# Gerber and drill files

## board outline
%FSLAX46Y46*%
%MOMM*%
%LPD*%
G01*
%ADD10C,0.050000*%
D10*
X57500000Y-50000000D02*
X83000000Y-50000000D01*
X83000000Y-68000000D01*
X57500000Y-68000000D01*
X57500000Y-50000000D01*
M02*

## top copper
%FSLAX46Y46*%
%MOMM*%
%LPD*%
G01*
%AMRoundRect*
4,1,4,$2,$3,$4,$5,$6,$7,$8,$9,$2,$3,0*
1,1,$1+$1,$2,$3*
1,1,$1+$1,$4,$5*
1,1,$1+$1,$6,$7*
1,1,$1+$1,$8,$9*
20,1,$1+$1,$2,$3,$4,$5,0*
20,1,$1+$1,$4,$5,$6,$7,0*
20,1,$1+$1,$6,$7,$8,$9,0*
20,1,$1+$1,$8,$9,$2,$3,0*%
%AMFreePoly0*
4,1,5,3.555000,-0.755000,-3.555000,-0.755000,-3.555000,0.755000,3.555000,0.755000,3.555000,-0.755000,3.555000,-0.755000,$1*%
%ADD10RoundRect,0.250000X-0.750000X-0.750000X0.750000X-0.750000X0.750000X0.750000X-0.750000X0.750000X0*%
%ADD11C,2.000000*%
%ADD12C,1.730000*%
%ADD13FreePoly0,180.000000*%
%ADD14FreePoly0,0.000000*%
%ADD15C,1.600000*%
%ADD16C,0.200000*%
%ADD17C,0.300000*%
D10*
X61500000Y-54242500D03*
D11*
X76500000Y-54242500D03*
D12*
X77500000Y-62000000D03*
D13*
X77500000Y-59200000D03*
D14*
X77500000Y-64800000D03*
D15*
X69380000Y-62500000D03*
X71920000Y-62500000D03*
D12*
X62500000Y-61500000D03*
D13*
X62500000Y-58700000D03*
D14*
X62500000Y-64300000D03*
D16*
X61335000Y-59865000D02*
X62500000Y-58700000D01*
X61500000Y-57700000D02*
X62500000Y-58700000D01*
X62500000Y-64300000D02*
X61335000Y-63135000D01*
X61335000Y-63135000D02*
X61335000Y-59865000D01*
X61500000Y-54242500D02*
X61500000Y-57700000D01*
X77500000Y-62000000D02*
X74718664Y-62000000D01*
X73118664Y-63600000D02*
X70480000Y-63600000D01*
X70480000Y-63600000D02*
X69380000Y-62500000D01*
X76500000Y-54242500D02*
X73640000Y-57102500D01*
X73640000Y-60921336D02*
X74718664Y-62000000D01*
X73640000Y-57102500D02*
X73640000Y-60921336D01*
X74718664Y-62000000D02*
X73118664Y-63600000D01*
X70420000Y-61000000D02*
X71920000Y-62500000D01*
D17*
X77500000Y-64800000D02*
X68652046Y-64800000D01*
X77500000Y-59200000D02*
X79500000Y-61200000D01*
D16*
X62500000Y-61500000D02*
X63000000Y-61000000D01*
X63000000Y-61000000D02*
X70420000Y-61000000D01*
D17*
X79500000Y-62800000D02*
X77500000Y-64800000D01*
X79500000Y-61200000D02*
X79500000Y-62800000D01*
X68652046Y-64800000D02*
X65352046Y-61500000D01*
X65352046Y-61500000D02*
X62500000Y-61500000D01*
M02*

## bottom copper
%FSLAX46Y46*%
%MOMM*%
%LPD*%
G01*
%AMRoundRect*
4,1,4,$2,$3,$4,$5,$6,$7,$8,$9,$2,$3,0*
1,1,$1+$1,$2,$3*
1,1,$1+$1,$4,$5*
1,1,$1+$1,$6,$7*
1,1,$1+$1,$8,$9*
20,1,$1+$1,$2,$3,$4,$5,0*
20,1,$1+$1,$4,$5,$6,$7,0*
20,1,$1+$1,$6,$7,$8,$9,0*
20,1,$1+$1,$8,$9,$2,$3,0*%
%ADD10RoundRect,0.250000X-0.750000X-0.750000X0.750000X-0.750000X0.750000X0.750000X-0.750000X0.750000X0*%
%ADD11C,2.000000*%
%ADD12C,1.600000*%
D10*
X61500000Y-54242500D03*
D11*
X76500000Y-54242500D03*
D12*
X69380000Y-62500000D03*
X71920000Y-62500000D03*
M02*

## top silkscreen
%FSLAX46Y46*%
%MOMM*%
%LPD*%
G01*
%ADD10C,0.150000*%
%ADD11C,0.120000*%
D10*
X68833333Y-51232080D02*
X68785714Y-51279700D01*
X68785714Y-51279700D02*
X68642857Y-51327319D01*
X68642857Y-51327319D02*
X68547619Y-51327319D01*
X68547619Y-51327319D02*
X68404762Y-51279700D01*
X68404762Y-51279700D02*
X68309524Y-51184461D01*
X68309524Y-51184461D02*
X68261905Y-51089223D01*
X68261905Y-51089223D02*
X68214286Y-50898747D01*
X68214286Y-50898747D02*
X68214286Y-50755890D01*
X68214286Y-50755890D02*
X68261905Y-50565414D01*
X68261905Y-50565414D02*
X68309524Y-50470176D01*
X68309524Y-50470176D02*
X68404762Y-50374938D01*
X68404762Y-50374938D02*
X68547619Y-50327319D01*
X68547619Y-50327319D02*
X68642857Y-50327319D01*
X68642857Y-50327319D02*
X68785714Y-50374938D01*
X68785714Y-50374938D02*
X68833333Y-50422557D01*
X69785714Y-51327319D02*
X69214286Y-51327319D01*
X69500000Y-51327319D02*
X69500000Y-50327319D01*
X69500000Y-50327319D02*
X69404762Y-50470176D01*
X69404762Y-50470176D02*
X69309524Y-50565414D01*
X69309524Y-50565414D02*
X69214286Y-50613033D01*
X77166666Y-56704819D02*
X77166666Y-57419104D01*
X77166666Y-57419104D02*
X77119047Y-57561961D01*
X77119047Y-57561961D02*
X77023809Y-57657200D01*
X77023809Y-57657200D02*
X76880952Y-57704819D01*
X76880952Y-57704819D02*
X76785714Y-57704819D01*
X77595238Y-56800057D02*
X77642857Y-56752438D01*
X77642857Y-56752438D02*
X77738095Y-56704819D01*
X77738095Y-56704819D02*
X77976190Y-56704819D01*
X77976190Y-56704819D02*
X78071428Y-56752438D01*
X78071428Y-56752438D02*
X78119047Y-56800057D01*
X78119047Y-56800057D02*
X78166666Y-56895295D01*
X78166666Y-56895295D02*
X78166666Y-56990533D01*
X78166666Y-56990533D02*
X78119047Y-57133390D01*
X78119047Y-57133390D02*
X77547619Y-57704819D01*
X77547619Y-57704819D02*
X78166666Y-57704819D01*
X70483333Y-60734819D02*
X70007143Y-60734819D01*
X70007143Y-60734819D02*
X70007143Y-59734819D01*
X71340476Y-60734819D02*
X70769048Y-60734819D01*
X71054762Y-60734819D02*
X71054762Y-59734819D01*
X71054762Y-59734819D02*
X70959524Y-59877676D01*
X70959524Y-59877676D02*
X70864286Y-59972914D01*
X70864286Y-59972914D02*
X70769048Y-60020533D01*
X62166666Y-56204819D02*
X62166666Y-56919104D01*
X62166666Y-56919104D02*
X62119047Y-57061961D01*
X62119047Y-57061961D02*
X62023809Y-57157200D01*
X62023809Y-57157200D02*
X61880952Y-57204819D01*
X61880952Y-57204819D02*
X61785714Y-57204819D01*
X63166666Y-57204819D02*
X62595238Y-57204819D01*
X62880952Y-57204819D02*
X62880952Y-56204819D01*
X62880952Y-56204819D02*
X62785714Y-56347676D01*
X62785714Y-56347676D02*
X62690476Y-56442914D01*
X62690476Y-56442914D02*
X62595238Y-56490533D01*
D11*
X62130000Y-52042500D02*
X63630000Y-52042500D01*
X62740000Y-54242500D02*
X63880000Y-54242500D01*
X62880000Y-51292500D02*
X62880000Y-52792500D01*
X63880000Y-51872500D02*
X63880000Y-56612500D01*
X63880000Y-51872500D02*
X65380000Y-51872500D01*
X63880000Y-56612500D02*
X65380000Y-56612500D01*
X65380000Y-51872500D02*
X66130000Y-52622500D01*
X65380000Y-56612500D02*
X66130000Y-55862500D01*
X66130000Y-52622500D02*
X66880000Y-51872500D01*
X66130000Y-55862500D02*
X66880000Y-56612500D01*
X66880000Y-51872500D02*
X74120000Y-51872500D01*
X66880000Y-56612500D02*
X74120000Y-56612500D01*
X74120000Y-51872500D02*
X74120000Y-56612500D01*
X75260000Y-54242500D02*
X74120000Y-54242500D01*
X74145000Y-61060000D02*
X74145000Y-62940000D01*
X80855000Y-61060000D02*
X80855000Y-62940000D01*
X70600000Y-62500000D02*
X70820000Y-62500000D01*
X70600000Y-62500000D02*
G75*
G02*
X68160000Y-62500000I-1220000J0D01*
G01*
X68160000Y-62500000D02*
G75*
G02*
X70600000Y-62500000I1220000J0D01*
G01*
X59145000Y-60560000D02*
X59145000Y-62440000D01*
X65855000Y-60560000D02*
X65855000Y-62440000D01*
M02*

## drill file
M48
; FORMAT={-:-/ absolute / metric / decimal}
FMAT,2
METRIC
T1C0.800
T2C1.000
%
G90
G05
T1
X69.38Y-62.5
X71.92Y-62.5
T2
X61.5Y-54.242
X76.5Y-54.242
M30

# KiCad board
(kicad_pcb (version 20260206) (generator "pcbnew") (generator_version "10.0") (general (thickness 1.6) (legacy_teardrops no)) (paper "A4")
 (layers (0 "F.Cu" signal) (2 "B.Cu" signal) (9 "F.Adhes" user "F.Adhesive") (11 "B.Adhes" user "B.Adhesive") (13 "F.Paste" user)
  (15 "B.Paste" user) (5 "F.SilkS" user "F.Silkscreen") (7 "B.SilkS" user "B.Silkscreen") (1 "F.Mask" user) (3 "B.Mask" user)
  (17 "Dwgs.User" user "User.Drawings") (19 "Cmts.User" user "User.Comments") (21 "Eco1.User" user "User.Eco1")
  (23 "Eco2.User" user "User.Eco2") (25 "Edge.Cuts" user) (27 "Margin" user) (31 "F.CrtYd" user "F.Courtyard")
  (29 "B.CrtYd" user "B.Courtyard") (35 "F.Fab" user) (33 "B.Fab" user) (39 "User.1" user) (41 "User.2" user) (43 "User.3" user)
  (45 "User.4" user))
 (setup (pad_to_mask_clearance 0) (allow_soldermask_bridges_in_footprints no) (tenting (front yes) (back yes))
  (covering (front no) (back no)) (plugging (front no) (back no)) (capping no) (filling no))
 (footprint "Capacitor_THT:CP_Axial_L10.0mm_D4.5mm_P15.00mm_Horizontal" (layer "F.Cu") (at 61.5 54.2425)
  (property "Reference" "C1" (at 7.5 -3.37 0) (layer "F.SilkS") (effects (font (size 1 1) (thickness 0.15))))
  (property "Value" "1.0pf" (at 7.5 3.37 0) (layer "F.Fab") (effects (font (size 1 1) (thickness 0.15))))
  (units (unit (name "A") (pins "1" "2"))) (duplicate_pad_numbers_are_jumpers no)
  (fp_line (start 0.63 -2.2) (end 2.13 -2.2) (stroke (width 0.12) (type solid)) (layer "F.SilkS"))
  (fp_line (start 1.24 0) (end 2.38 0) (stroke (width 0.12) (type solid)) (layer "F.SilkS"))
  (fp_line (start 1.38 -2.95) (end 1.38 -1.45) (stroke (width 0.12) (type solid)) (layer "F.SilkS"))
  (fp_line (start 2.38 -2.37) (end 2.38 2.37) (stroke (width 0.12) (type solid)) (layer "F.SilkS"))
  (fp_line (start 2.38 -2.37) (end 3.88 -2.37) (stroke (width 0.12) (type solid)) (layer "F.SilkS"))
  (fp_line (start 2.38 2.37) (end 3.88 2.37) (stroke (width 0.12) (type solid)) (layer "F.SilkS"))
  (fp_line (start 3.88 -2.37) (end 4.63 -1.62) (stroke (width 0.12) (type solid)) (layer "F.SilkS"))
  (fp_line (start 3.88 2.37) (end 4.63 1.62) (stroke (width 0.12) (type solid)) (layer "F.SilkS"))
  (fp_line (start 4.63 -1.62) (end 5.38 -2.37) (stroke (width 0.12) (type solid)) (layer "F.SilkS"))
  (fp_line (start 4.63 1.62) (end 5.38 2.37) (stroke (width 0.12) (type solid)) (layer "F.SilkS"))
  (fp_line (start 5.38 -2.37) (end 12.62 -2.37) (stroke (width 0.12) (type solid)) (layer "F.SilkS"))
  (fp_line (start 5.38 2.37) (end 12.62 2.37) (stroke (width 0.12) (type solid)) (layer "F.SilkS"))
  (fp_line (start 12.62 -2.37) (end 12.62 2.37) (stroke (width 0.12) (type solid)) (layer "F.SilkS"))
  (fp_line (start 13.76 0) (end 12.62 0) (stroke (width 0.12) (type solid)) (layer "F.SilkS"))
  (pad "1" thru_hole roundrect (at 0 0) (size 2 2) (drill 1) (layers "*.Cu" "*.Mask") (remove_unused_layers no) (roundrect_rratio 0.125)
   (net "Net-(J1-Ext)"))
  (pad "2" thru_hole circle (at 15 0) (size 2 2) (drill 1) (layers "*.Cu" "*.Mask") (remove_unused_layers no) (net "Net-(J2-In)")))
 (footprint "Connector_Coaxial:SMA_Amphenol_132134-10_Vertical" (layer "F.Cu") (at 77.5 62)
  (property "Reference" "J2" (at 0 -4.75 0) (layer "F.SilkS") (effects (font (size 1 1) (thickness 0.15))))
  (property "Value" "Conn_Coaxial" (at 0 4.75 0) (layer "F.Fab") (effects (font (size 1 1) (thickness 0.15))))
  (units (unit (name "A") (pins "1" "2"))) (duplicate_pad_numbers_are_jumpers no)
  (fp_line (start -3.355 -0.94) (end -3.355 0.94) (stroke (width 0.12) (type solid)) (layer "F.SilkS"))
  (fp_line (start 3.355 -0.94) (end 3.355 0.94) (stroke (width 0.12) (type solid)) (layer "F.SilkS"))
  (pad "1" smd circle (at 0 0 90) (size 1.73 1.73) (layers "F.Cu" "F.Mask" "F.Paste") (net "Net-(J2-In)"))
  (pad "2" smd custom (at 0 -2.8 180) (size 7.11 1.51) (layers "F.Cu" "F.Mask" "F.Paste") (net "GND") (zone_connect 2)
   (options (clearance outline) (anchor rect)) (primitives))
  (pad "2" smd custom (at 0 2.8) (size 7.11 1.51) (layers "F.Cu" "F.Mask" "F.Paste") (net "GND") (zone_connect 2)
   (options (clearance outline) (anchor rect)) (primitives)))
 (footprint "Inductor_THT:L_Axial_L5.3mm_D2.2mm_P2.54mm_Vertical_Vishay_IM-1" (layer "F.Cu") (at 69.38 62.5)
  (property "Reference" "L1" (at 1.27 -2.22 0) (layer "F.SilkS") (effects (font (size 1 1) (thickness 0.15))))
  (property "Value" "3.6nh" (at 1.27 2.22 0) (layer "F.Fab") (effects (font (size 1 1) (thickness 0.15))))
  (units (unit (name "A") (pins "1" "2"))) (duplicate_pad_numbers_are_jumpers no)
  (fp_line (start 1.22 0) (end 1.44 0) (stroke (width 0.12) (type solid)) (layer "F.SilkS"))
  (fp_circle (center 0 0) (end 1.22 0) (stroke (width 0.12) (type solid)) (fill no) (layer "F.SilkS"))
  (pad "1" thru_hole circle (at 0 0) (size 1.6 1.6) (drill 0.8) (layers "*.Cu" "*.Mask") (remove_unused_layers no) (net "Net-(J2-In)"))
  (pad "2" thru_hole circle (at 2.54 0) (size 1.6 1.6) (drill 0.8) (layers "*.Cu" "*.Mask") (remove_unused_layers no) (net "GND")))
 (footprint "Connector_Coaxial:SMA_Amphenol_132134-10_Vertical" (layer "F.Cu") (at 62.5 61.5)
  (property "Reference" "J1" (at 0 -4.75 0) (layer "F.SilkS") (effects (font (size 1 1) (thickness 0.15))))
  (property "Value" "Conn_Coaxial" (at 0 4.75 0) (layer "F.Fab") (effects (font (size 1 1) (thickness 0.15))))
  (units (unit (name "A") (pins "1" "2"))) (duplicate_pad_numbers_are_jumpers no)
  (fp_line (start -3.355 -0.94) (end -3.355 0.94) (stroke (width 0.12) (type solid)) (layer "F.SilkS"))
  (fp_line (start 3.355 -0.94) (end 3.355 0.94) (stroke (width 0.12) (type solid)) (layer "F.SilkS"))
  (pad "1" smd circle (at 0 0 90) (size 1.73 1.73) (layers "F.Cu" "F.Mask" "F.Paste") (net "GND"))
  (pad "2" smd custom (at 0 -2.8 180) (size 7.11 1.51) (layers "F.Cu" "F.Mask" "F.Paste") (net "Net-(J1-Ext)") (zone_connect 2)
   (options (clearance outline) (anchor rect)) (primitives))
  (pad "2" smd custom (at 0 2.8) (size 7.11 1.51) (layers "F.Cu" "F.Mask" "F.Paste") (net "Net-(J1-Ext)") (zone_connect 2)
   (options (clearance outline) (anchor rect)) (primitives)))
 (gr_rect (start 57.5 50) (end 83 68) (stroke (width 0.05) (type default)) (fill no) (layer "Edge.Cuts"))
 (segment (start 61.335 59.865) (end 62.5 58.7) (width 0.2) (layer "F.Cu") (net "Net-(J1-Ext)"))
 (segment (start 61.5 57.7) (end 62.5 58.7) (width 0.2) (layer "F.Cu") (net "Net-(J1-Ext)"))
 (segment (start 62.5 64.3) (end 61.335 63.135) (width 0.2) (layer "F.Cu") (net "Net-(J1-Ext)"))
 (segment (start 61.335 63.135) (end 61.335 59.865) (width 0.2) (layer "F.Cu") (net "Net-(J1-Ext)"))
 (segment (start 61.5 54.2425) (end 61.5 57.7) (width 0.2) (layer "F.Cu") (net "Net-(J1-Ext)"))
 (segment (start 77.5 62) (end 74.718664 62) (width 0.2) (layer "F.Cu") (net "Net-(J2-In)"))
 (segment (start 73.118664 63.6) (end 70.48 63.6) (width 0.2) (layer "F.Cu") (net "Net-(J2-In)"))
 (segment (start 70.48 63.6) (end 69.38 62.5) (width 0.2) (layer "F.Cu") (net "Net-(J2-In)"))
 (segment (start 76.5 54.2425) (end 73.64 57.1025) (width 0.2) (layer "F.Cu") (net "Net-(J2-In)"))
 (segment (start 73.64 60.921336) (end 74.718664 62) (width 0.2) (layer "F.Cu") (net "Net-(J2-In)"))
 (segment (start 73.64 57.1025) (end 73.64 60.921336) (width 0.2) (layer "F.Cu") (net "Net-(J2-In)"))
 (segment (start 74.718664 62) (end 73.118664 63.6) (width 0.2) (layer "F.Cu") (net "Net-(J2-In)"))
 (segment (start 70.42 61) (end 71.92 62.5) (width 0.2) (layer "F.Cu") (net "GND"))
 (segment (start 77.5 64.8) (end 68.652046 64.8) (width 0.3) (layer "F.Cu") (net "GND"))
 (segment (start 77.5 59.2) (end 79.5 61.2) (width 0.3) (layer "F.Cu") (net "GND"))
 (segment (start 62.5 61.5) (end 63 61) (width 0.2) (layer "F.Cu") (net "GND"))
 (segment (start 63 61) (end 70.42 61) (width 0.2) (layer "F.Cu") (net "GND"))
 (segment (start 79.5 62.8) (end 77.5 64.8) (width 0.3) (layer "F.Cu") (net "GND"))
 (segment (start 79.5 61.2) (end 79.5 62.8) (width 0.3) (layer "F.Cu") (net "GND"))
 (segment (start 68.652046 64.8) (end 65.352046 61.5) (width 0.3) (layer "F.Cu") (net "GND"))
 (segment (start 65.352046 61.5) (end 62.5 61.5) (width 0.3) (layer "F.Cu") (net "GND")))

